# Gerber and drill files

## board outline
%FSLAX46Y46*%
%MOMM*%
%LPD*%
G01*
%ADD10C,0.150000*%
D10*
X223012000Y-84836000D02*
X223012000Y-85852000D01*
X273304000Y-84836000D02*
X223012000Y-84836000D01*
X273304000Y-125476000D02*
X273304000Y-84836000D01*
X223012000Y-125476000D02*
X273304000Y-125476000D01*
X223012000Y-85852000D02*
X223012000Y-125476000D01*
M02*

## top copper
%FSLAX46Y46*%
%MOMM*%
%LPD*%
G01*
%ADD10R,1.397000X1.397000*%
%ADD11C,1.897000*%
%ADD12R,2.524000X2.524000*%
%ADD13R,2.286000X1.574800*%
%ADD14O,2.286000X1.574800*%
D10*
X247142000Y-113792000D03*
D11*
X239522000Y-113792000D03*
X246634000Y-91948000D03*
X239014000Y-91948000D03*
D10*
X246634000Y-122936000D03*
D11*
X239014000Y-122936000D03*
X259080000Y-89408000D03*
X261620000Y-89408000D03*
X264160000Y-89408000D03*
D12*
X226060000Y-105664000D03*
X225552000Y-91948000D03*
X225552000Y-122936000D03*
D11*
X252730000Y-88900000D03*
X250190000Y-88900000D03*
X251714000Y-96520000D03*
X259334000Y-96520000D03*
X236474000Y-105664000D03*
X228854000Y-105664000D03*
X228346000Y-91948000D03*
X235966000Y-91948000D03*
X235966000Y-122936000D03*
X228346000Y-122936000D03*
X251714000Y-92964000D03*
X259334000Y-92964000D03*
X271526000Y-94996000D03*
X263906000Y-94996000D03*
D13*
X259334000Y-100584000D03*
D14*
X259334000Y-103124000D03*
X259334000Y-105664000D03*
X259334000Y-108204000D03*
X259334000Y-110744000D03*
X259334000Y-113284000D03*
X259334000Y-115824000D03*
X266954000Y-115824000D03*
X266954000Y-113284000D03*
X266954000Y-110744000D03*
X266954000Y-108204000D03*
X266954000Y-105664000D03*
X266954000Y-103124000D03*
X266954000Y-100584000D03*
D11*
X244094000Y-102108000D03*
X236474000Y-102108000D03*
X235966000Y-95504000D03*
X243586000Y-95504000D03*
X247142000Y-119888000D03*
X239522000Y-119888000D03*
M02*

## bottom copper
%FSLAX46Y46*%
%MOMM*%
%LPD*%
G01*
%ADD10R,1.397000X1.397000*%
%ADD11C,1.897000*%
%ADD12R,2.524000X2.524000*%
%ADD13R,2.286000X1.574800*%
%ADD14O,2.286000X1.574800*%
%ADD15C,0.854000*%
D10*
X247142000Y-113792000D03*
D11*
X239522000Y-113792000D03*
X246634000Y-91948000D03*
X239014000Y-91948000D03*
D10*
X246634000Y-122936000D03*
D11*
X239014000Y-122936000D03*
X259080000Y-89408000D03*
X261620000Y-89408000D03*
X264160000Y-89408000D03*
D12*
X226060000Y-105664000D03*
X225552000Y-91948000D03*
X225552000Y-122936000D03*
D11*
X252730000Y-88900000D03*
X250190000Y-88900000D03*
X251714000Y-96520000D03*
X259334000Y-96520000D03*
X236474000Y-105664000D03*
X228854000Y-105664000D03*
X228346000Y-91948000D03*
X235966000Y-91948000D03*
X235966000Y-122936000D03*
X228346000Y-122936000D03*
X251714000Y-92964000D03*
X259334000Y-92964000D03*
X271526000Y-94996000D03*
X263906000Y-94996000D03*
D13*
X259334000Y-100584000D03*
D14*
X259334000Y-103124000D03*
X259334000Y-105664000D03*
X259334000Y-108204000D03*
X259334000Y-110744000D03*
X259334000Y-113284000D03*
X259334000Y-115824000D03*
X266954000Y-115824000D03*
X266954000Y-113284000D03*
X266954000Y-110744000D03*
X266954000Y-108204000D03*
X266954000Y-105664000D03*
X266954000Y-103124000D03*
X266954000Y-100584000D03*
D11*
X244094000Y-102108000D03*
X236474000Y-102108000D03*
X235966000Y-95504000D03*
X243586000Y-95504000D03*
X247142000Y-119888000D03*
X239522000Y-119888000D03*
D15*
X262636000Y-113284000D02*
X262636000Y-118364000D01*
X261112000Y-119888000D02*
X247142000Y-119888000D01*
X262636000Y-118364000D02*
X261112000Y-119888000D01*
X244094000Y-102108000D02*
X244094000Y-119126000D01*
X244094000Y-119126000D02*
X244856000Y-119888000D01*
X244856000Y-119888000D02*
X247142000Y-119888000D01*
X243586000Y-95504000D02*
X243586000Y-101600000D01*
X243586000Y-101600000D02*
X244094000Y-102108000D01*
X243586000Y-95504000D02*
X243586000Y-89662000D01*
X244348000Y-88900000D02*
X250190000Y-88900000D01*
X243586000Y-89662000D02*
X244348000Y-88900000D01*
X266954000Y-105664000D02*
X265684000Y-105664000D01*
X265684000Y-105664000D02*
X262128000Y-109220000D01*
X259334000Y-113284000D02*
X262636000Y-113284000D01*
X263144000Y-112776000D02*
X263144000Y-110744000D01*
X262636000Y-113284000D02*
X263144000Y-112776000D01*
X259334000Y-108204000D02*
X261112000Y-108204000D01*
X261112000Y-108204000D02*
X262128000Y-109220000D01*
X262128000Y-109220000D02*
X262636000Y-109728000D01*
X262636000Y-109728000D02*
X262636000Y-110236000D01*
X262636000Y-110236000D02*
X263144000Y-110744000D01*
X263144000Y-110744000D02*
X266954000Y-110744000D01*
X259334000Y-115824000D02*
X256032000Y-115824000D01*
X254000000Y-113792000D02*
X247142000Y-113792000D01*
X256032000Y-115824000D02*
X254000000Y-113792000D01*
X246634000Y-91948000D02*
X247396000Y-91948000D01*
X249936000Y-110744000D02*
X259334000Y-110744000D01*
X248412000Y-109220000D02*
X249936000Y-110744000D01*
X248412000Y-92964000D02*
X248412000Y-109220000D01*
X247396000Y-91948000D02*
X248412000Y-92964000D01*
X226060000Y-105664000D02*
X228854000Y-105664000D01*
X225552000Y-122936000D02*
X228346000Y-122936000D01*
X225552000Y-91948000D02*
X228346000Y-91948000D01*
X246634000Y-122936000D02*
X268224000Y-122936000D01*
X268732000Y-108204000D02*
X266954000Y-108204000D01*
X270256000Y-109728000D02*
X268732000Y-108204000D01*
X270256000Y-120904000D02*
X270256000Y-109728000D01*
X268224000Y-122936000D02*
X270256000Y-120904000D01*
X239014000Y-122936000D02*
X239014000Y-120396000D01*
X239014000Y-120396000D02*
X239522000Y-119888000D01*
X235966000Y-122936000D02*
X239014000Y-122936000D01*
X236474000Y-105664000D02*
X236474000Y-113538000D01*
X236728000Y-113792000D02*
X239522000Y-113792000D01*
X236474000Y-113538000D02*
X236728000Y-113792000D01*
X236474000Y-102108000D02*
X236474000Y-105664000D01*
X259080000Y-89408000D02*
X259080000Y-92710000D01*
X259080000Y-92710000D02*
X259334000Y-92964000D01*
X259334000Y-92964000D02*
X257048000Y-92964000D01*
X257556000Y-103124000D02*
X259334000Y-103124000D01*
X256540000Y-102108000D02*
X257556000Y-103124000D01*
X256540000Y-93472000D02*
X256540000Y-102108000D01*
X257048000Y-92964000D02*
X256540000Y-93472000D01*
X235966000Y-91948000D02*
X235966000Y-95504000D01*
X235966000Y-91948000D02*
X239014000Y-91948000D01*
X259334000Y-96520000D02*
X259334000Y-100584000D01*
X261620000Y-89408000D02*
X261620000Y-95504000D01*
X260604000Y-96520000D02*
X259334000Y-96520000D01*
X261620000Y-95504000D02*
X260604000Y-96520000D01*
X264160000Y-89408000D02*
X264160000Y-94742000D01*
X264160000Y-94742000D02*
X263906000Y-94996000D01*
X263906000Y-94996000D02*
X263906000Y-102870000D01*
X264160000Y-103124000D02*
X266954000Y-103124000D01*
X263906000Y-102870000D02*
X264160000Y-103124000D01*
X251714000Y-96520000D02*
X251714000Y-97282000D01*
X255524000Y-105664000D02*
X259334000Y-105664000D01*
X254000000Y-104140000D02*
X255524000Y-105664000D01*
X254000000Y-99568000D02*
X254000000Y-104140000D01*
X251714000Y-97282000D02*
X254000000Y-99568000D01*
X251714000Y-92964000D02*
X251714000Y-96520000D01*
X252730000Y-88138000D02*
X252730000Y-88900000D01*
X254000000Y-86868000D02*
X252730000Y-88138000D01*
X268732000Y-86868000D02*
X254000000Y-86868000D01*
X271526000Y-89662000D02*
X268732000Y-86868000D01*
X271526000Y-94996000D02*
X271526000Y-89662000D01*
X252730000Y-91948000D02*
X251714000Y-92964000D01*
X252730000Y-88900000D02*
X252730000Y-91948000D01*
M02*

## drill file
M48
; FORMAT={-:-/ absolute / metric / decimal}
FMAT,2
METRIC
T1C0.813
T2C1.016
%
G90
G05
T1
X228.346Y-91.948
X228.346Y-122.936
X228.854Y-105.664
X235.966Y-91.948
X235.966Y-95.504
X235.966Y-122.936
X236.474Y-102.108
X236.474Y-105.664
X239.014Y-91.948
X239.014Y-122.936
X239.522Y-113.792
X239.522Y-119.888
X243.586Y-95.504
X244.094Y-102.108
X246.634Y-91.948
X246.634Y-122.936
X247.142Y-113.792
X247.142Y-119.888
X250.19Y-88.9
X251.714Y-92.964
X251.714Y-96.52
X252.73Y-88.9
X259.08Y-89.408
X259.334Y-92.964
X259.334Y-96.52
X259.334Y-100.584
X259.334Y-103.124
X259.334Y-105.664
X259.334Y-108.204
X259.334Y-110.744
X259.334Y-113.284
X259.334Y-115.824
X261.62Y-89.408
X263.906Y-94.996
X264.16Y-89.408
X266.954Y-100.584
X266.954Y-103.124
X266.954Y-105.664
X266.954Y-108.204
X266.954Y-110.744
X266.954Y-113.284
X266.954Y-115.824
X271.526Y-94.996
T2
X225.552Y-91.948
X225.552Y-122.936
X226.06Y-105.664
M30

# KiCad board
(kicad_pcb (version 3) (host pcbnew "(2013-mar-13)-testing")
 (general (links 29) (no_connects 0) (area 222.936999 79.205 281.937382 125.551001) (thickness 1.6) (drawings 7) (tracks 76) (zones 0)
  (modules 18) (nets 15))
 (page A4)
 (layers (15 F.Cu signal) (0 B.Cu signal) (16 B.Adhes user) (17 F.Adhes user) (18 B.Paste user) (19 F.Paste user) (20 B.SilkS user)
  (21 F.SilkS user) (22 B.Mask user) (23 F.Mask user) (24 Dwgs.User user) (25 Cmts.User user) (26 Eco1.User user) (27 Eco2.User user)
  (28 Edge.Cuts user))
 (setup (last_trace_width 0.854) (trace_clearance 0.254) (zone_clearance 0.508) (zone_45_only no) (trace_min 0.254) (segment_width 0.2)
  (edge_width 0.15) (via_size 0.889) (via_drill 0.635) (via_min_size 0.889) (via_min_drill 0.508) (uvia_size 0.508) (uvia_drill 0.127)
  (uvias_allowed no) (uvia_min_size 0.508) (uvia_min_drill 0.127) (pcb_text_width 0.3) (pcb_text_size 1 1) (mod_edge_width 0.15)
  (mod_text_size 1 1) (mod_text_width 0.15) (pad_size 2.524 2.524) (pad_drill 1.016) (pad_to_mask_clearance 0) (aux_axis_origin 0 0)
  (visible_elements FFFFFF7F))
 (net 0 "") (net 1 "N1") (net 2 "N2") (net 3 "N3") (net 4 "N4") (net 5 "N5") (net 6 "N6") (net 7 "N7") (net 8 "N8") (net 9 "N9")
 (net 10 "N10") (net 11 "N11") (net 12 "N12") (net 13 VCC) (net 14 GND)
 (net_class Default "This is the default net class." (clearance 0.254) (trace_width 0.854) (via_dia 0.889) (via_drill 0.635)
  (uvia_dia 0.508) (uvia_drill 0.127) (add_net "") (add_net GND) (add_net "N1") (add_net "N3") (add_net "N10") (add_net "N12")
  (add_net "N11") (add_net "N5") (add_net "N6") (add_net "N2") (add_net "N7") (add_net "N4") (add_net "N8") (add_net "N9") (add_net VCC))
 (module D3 (layer F.Cu) (at 243.332 113.792)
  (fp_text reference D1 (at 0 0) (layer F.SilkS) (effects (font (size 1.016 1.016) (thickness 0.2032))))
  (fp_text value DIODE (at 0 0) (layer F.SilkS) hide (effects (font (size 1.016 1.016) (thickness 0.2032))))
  (pad 2 thru_hole rect (at 3.81 0) (size 1.397 1.397) (drill 0.8128) (layers *.Cu *.Mask F.SilkS) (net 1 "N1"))
  (pad 1 thru_hole circle (at -3.81 0) (size 1.897 1.897) (drill 0.8128) (layers *.Cu *.Mask F.SilkS) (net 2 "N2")))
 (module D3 (layer F.Cu) (at 242.824 91.948)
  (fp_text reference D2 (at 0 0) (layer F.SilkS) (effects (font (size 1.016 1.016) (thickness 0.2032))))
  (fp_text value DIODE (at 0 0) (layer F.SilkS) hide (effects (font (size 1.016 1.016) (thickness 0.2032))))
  (pad 2 thru_hole circle (at 3.81 0) (size 1.897 1.897) (drill 0.8128) (layers *.Cu *.Mask F.SilkS) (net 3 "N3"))
  (pad 1 thru_hole circle (at -3.81 0) (size 1.897 1.897) (drill 0.8128) (layers *.Cu *.Mask F.SilkS) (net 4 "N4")))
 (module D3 (layer F.Cu) (at 242.824 122.936)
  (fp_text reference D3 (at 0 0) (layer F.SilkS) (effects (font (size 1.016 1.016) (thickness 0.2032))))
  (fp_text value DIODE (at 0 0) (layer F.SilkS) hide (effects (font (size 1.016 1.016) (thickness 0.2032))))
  (pad 2 thru_hole rect (at 3.81 0) (size 1.397 1.397) (drill 0.8128) (layers *.Cu *.Mask F.SilkS) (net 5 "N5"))
  (pad 1 thru_hole circle (at -3.81 0) (size 1.897 1.897) (drill 0.8128) (layers *.Cu *.Mask F.SilkS) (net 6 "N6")))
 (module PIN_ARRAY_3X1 (layer F.Cu) (at 261.62 89.408)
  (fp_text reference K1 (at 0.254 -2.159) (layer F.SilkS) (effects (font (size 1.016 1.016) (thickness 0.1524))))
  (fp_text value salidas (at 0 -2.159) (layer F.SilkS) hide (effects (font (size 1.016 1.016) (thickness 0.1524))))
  (pad 1 thru_hole circle (at -2.54 0) (size 1.897 1.897) (drill 0.8128) (layers *.Cu *.Mask F.SilkS) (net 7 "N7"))
  (pad 2 thru_hole circle (at 0 0) (size 1.897 1.897) (drill 0.8128) (layers *.Cu *.Mask F.SilkS) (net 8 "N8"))
  (pad 3 thru_hole circle (at 2.54 0) (size 1.897 1.897) (drill 0.8128) (layers *.Cu *.Mask F.SilkS) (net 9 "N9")))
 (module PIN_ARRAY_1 (layer F.Cu) (at 226.06 105.664)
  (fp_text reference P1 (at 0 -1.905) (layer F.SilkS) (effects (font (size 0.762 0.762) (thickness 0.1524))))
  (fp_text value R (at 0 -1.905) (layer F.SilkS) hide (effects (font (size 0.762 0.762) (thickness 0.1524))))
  (pad 1 thru_hole rect (at 0 0) (size 2.524 2.524) (drill 1.016) (layers *.Cu *.Mask F.SilkS) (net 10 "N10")))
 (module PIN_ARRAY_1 (layer F.Cu) (at 225.552 91.948)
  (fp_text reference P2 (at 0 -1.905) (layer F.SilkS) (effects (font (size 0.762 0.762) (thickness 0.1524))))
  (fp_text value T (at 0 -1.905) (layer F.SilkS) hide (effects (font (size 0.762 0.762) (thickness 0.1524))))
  (pad 1 thru_hole rect (at 0 0) (size 2.524 2.524) (drill 1.016) (layers *.Cu *.Mask F.SilkS) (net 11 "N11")))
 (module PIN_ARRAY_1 (layer F.Cu) (at 225.552 122.936)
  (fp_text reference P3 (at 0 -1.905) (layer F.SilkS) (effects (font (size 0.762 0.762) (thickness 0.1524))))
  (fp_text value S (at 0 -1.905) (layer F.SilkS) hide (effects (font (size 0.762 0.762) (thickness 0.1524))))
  (pad 1 thru_hole rect (at 0 0) (size 2.524 2.524) (drill 1.016) (layers *.Cu *.Mask F.SilkS) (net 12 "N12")))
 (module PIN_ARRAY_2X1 (layer F.Cu) (at 251.46 88.9 180)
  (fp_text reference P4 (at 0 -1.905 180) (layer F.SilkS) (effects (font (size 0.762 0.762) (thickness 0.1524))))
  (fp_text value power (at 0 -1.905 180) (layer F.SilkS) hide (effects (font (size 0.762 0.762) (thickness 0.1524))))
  (pad 1 thru_hole circle (at -1.27 0 180) (size 1.897 1.897) (drill 0.8128) (layers *.Cu *.Mask F.SilkS) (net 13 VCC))
  (pad 2 thru_hole circle (at 1.27 0 180) (size 1.897 1.897) (drill 0.8128) (layers *.Cu *.Mask F.SilkS) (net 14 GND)))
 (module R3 (layer F.Cu) (at 255.524 96.52) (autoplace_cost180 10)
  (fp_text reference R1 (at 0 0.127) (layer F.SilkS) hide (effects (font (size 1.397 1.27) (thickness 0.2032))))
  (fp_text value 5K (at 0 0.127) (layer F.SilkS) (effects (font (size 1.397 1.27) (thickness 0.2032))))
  (pad 1 thru_hole circle (at -3.81 0) (size 1.897 1.897) (drill 0.8128) (layers *.Cu *.Mask F.SilkS) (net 13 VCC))
  (pad 2 thru_hole circle (at 3.81 0) (size 1.897 1.897) (drill 0.8128) (layers *.Cu *.Mask F.SilkS) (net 8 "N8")))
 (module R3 (layer F.Cu) (at 232.664 105.664 180) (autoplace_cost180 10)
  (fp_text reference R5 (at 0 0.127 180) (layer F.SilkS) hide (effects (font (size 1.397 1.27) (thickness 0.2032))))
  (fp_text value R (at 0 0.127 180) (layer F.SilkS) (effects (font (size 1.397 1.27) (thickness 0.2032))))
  (pad 1 thru_hole circle (at -3.81 0 180) (size 1.897 1.897) (drill 0.8128) (layers *.Cu *.Mask F.SilkS) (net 2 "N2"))
  (pad 2 thru_hole circle (at 3.81 0 180) (size 1.897 1.897) (drill 0.8128) (layers *.Cu *.Mask F.SilkS) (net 10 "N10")))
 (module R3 (layer F.Cu) (at 232.156 91.948) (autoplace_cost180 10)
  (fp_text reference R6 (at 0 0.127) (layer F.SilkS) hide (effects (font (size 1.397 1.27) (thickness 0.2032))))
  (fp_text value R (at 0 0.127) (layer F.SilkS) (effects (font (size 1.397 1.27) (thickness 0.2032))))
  (pad 1 thru_hole circle (at -3.81 0) (size 1.897 1.897) (drill 0.8128) (layers *.Cu *.Mask F.SilkS) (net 11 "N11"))
  (pad 2 thru_hole circle (at 3.81 0) (size 1.897 1.897) (drill 0.8128) (layers *.Cu *.Mask F.SilkS) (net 4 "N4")))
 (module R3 (layer F.Cu) (at 232.156 122.936 180) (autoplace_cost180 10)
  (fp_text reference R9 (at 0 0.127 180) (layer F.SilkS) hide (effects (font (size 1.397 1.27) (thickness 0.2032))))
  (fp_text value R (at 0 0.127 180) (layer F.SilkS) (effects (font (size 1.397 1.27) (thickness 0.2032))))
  (pad 1 thru_hole circle (at -3.81 0 180) (size 1.897 1.897) (drill 0.8128) (layers *.Cu *.Mask F.SilkS) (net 6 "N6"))
  (pad 2 thru_hole circle (at 3.81 0 180) (size 1.897 1.897) (drill 0.8128) (layers *.Cu *.Mask F.SilkS) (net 12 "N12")))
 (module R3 (layer F.Cu) (at 255.524 92.964) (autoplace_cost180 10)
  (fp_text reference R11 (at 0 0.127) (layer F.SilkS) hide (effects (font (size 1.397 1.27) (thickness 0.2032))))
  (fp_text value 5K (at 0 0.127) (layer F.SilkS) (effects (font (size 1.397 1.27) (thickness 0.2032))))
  (pad 1 thru_hole circle (at -3.81 0) (size 1.897 1.897) (drill 0.8128) (layers *.Cu *.Mask F.SilkS) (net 13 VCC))
  (pad 2 thru_hole circle (at 3.81 0) (size 1.897 1.897) (drill 0.8128) (layers *.Cu *.Mask F.SilkS) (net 7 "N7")))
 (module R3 (layer F.Cu) (at 267.716 94.996 180) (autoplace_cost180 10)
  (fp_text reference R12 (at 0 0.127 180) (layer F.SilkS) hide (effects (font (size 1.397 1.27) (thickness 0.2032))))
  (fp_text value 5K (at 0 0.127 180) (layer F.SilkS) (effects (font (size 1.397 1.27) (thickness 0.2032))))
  (pad 1 thru_hole circle (at -3.81 0 180) (size 1.897 1.897) (drill 0.8128) (layers *.Cu *.Mask F.SilkS) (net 13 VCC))
  (pad 2 thru_hole circle (at 3.81 0 180) (size 1.897 1.897) (drill 0.8128) (layers *.Cu *.Mask F.SilkS) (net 9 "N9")))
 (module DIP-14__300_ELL (layer F.Cu) (at 263.144 108.204 270)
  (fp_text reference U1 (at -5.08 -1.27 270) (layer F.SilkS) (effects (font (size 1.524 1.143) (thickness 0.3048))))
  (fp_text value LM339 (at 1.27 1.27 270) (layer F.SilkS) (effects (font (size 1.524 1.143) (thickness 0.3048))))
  (pad 1 thru_hole rect (at -7.62 3.81 270) (size 1.5748 2.286) (drill 0.8128) (layers *.Cu *.Mask F.SilkS) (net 8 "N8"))
  (pad 2 thru_hole oval (at -5.08 3.81 270) (size 1.5748 2.286) (drill 0.8128) (layers *.Cu *.Mask F.SilkS) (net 7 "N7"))
  (pad 3 thru_hole oval (at -2.54 3.81 270) (size 1.5748 2.286) (drill 0.8128) (layers *.Cu *.Mask F.SilkS) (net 13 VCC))
  (pad 4 thru_hole oval (at 0 3.81 270) (size 1.5748 2.286) (drill 0.8128) (layers *.Cu *.Mask F.SilkS) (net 14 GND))
  (pad 5 thru_hole oval (at 2.54 3.81 270) (size 1.5748 2.286) (drill 0.8128) (layers *.Cu *.Mask F.SilkS) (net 3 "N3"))
  (pad 6 thru_hole oval (at 5.08 3.81 270) (size 1.5748 2.286) (drill 0.8128) (layers *.Cu *.Mask F.SilkS) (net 14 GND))
  (pad 7 thru_hole oval (at 7.62 3.81 270) (size 1.5748 2.286) (drill 0.8128) (layers *.Cu *.Mask F.SilkS) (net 1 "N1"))
  (pad 8 thru_hole oval (at 7.62 -3.81 270) (size 1.5748 2.286) (drill 0.8128) (layers *.Cu *.Mask F.SilkS))
  (pad 9 thru_hole oval (at 5.08 -3.81 270) (size 1.5748 2.286) (drill 0.8128) (layers *.Cu *.Mask F.SilkS))
  (pad 10 thru_hole oval (at 2.54 -3.81 270) (size 1.5748 2.286) (drill 0.8128) (layers *.Cu *.Mask F.SilkS) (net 14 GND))
  (pad 11 thru_hole oval (at 0 -3.81 270) (size 1.5748 2.286) (drill 0.8128) (layers *.Cu *.Mask F.SilkS) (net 5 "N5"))
  (pad 12 thru_hole oval (at -2.54 -3.81 270) (size 1.5748 2.286) (drill 0.8128) (layers *.Cu *.Mask F.SilkS) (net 14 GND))
  (pad 13 thru_hole oval (at -5.08 -3.81 270) (size 1.5748 2.286) (drill 0.8128) (layers *.Cu *.Mask F.SilkS) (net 9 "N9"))
  (pad 14 thru_hole oval (at -7.62 -3.81 270) (size 1.5748 2.286) (drill 0.8128) (layers *.Cu *.Mask F.SilkS)))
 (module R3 (layer F.Cu) (at 240.284 102.108 180) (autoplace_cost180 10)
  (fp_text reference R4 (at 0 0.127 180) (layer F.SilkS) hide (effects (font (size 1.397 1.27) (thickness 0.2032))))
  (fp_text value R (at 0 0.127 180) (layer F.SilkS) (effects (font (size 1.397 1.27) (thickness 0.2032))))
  (pad 1 thru_hole circle (at -3.81 0 180) (size 1.897 1.897) (drill 0.8128) (layers *.Cu *.Mask F.SilkS) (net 14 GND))
  (pad 2 thru_hole circle (at 3.81 0 180) (size 1.897 1.897) (drill 0.8128) (layers *.Cu *.Mask F.SilkS) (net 2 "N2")))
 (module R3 (layer F.Cu) (at 239.776 95.504) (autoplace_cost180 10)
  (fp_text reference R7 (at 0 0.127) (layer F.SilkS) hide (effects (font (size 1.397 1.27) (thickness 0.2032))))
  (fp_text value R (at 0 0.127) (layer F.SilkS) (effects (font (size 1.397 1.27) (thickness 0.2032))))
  (pad 1 thru_hole circle (at -3.81 0) (size 1.897 1.897) (drill 0.8128) (layers *.Cu *.Mask F.SilkS) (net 4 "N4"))
  (pad 2 thru_hole circle (at 3.81 0) (size 1.897 1.897) (drill 0.8128) (layers *.Cu *.Mask F.SilkS) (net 14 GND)))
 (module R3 (layer F.Cu) (at 243.332 119.888 180) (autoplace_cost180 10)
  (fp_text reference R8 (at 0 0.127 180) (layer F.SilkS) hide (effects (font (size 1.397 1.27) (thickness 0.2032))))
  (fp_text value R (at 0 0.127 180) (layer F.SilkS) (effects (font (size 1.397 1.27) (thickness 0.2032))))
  (pad 1 thru_hole circle (at -3.81 0 180) (size 1.897 1.897) (drill 0.8128) (layers *.Cu *.Mask F.SilkS) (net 14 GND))
  (pad 2 thru_hole circle (at 3.81 0 180) (size 1.897 1.897) (drill 0.8128) (layers *.Cu *.Mask F.SilkS) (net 6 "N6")))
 (gr_line (start 223.012 84.836) (end 223.012 85.852) (angle 90) (layer Edge.Cuts) (width 0.15))
 (gr_line (start 273.304 84.836) (end 223.012 84.836) (angle 90) (layer Edge.Cuts) (width 0.15))
 (gr_line (start 273.304 125.476) (end 273.304 84.836) (angle 90) (layer Edge.Cuts) (width 0.15))
 (gr_line (start 223.012 125.476) (end 273.304 125.476) (angle 90) (layer Edge.Cuts) (width 0.15))
 (gr_line (start 223.012 85.852) (end 223.012 125.476) (angle 90) (layer Edge.Cuts) (width 0.15))
 (segment (start 262.636 113.284) (end 262.636 118.364) (width 0.854) (layer B.Cu) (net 14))
 (segment (start 261.112 119.888) (end 247.142 119.888) (width 0.854) (layer B.Cu) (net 14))
 (segment (start 262.636 118.364) (end 261.112 119.888) (width 0.854) (layer B.Cu) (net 14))
 (segment (start 244.094 102.108) (end 244.094 119.126) (width 0.854) (layer B.Cu) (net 14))
 (segment (start 244.094 119.126) (end 244.856 119.888) (width 0.854) (layer B.Cu) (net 14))
 (segment (start 244.856 119.888) (end 247.142 119.888) (width 0.854) (layer B.Cu) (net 14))
 (segment (start 243.586 95.504) (end 243.586 101.6) (width 0.854) (layer B.Cu) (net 14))
 (segment (start 243.586 101.6) (end 244.094 102.108) (width 0.854) (layer B.Cu) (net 14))
 (segment (start 243.586 95.504) (end 243.586 89.662) (width 0.854) (layer B.Cu) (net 14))
 (segment (start 244.348 88.9) (end 250.19 88.9) (width 0.854) (layer B.Cu) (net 14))
 (segment (start 243.586 89.662) (end 244.348 88.9) (width 0.854) (layer B.Cu) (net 14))
 (segment (start 266.954 105.664) (end 265.684 105.664) (width 0.854) (layer B.Cu) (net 14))
 (segment (start 265.684 105.664) (end 262.128 109.22) (width 0.854) (layer B.Cu) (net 14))
 (segment (start 259.334 113.284) (end 262.636 113.284) (width 0.854) (layer B.Cu) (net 14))
 (segment (start 263.144 112.776) (end 263.144 110.744) (width 0.854) (layer B.Cu) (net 14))
 (segment (start 262.636 113.284) (end 263.144 112.776) (width 0.854) (layer B.Cu) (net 14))
 (segment (start 259.334 108.204) (end 261.112 108.204) (width 0.854) (layer B.Cu) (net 14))
 (segment (start 261.112 108.204) (end 262.128 109.22) (width 0.854) (layer B.Cu) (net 14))
 (segment (start 262.128 109.22) (end 262.636 109.728) (width 0.854) (layer B.Cu) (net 14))
 (segment (start 262.636 109.728) (end 262.636 110.236) (width 0.854) (layer B.Cu) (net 14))
 (segment (start 262.636 110.236) (end 263.144 110.744) (width 0.854) (layer B.Cu) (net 14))
 (segment (start 263.144 110.744) (end 266.954 110.744) (width 0.854) (layer B.Cu) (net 14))
 (segment (start 259.334 115.824) (end 256.032 115.824) (width 0.854) (layer B.Cu) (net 1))
 (segment (start 254 113.792) (end 247.142 113.792) (width 0.854) (layer B.Cu) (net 1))
 (segment (start 256.032 115.824) (end 254 113.792) (width 0.854) (layer B.Cu) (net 1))
 (segment (start 246.634 91.948) (end 247.396 91.948) (width 0.854) (layer B.Cu) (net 3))
 (segment (start 249.936 110.744) (end 259.334 110.744) (width 0.854) (layer B.Cu) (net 3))
 (segment (start 248.412 109.22) (end 249.936 110.744) (width 0.854) (layer B.Cu) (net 3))
 (segment (start 248.412 92.964) (end 248.412 109.22) (width 0.854) (layer B.Cu) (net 3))
 (segment (start 247.396 91.948) (end 248.412 92.964) (width 0.854) (layer B.Cu) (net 3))
 (segment (start 226.06 105.664) (end 228.854 105.664) (width 0.854) (layer B.Cu) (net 10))
 (segment (start 225.552 122.936) (end 228.346 122.936) (width 0.854) (layer B.Cu) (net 12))
 (segment (start 225.552 91.948) (end 228.346 91.948) (width 0.854) (layer B.Cu) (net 11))
 (segment (start 246.634 122.936) (end 268.224 122.936) (width 0.854) (layer B.Cu) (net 5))
 (segment (start 268.732 108.204) (end 266.954 108.204) (width 0.854) (layer B.Cu) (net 5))
 (segment (start 270.256 109.728) (end 268.732 108.204) (width 0.854) (layer B.Cu) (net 5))
 (segment (start 270.256 120.904) (end 270.256 109.728) (width 0.854) (layer B.Cu) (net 5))
 (segment (start 268.224 122.936) (end 270.256 120.904) (width 0.854) (layer B.Cu) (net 5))
 (segment (start 239.014 122.936) (end 239.014 120.396) (width 0.854) (layer B.Cu) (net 6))
 (segment (start 239.014 120.396) (end 239.522 119.888) (width 0.854) (layer B.Cu) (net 6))
 (segment (start 235.966 122.936) (end 239.014 122.936) (width 0.854) (layer B.Cu) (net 6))
 (segment (start 236.474 105.664) (end 236.474 113.538) (width 0.854) (layer B.Cu) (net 2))
 (segment (start 236.728 113.792) (end 239.522 113.792) (width 0.854) (layer B.Cu) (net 2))
 (segment (start 236.474 113.538) (end 236.728 113.792) (width 0.854) (layer B.Cu) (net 2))
 (segment (start 236.474 102.108) (end 236.474 105.664) (width 0.854) (layer B.Cu) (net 2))
 (segment (start 259.08 89.408) (end 259.08 92.71) (width 0.854) (layer B.Cu) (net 7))
 (segment (start 259.08 92.71) (end 259.334 92.964) (width 0.854) (layer B.Cu) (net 7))
 (segment (start 259.334 92.964) (end 257.048 92.964) (width 0.854) (layer B.Cu) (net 7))
 (segment (start 257.556 103.124) (end 259.334 103.124) (width 0.854) (layer B.Cu) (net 7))
 (segment (start 256.54 102.108) (end 257.556 103.124) (width 0.854) (layer B.Cu) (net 7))
 (segment (start 256.54 93.472) (end 256.54 102.108) (width 0.854) (layer B.Cu) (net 7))
 (segment (start 257.048 92.964) (end 256.54 93.472) (width 0.854) (layer B.Cu) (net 7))
 (segment (start 235.966 91.948) (end 235.966 95.504) (width 0.854) (layer B.Cu) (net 4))
 (segment (start 235.966 91.948) (end 239.014 91.948) (width 0.854) (layer B.Cu) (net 4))
 (segment (start 259.334 96.52) (end 259.334 100.584) (width 0.854) (layer B.Cu) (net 8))
 (segment (start 261.62 89.408) (end 261.62 95.504) (width 0.854) (layer B.Cu) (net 8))
 (segment (start 260.604 96.52) (end 259.334 96.52) (width 0.854) (layer B.Cu) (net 8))
 (segment (start 261.62 95.504) (end 260.604 96.52) (width 0.854) (layer B.Cu) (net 8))
 (segment (start 264.16 89.408) (end 264.16 94.742) (width 0.854) (layer B.Cu) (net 9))
 (segment (start 264.16 94.742) (end 263.906 94.996) (width 0.854) (layer B.Cu) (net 9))
 (segment (start 263.906 94.996) (end 263.906 102.87) (width 0.854) (layer B.Cu) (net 9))
 (segment (start 264.16 103.124) (end 266.954 103.124) (width 0.854) (layer B.Cu) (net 9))
 (segment (start 263.906 102.87) (end 264.16 103.124) (width 0.854) (layer B.Cu) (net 9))
 (segment (start 251.714 96.52) (end 251.714 97.282) (width 0.854) (layer B.Cu) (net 13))
 (segment (start 255.524 105.664) (end 259.334 105.664) (width 0.854) (layer B.Cu) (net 13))
 (segment (start 254 104.14) (end 255.524 105.664) (width 0.854) (layer B.Cu) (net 13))
 (segment (start 254 99.568) (end 254 104.14) (width 0.854) (layer B.Cu) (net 13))
 (segment (start 251.714 97.282) (end 254 99.568) (width 0.854) (layer B.Cu) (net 13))
 (segment (start 251.714 92.964) (end 251.714 96.52) (width 0.854) (layer B.Cu) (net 13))
 (segment (start 252.73 88.138) (end 252.73 88.9) (width 0.854) (layer B.Cu) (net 13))
 (segment (start 254 86.868) (end 252.73 88.138) (width 0.854) (layer B.Cu) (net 13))
 (segment (start 268.732 86.868) (end 254 86.868) (width 0.854) (layer B.Cu) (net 13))
 (segment (start 271.526 89.662) (end 268.732 86.868) (width 0.854) (layer B.Cu) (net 13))
 (segment (start 271.526 94.996) (end 271.526 89.662) (width 0.854) (layer B.Cu) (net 13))
 (segment (start 252.73 91.948) (end 251.714 92.964) (width 0.854) (layer B.Cu) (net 13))
 (segment (start 252.73 88.9) (end 252.73 91.948) (width 0.854) (layer B.Cu) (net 13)))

